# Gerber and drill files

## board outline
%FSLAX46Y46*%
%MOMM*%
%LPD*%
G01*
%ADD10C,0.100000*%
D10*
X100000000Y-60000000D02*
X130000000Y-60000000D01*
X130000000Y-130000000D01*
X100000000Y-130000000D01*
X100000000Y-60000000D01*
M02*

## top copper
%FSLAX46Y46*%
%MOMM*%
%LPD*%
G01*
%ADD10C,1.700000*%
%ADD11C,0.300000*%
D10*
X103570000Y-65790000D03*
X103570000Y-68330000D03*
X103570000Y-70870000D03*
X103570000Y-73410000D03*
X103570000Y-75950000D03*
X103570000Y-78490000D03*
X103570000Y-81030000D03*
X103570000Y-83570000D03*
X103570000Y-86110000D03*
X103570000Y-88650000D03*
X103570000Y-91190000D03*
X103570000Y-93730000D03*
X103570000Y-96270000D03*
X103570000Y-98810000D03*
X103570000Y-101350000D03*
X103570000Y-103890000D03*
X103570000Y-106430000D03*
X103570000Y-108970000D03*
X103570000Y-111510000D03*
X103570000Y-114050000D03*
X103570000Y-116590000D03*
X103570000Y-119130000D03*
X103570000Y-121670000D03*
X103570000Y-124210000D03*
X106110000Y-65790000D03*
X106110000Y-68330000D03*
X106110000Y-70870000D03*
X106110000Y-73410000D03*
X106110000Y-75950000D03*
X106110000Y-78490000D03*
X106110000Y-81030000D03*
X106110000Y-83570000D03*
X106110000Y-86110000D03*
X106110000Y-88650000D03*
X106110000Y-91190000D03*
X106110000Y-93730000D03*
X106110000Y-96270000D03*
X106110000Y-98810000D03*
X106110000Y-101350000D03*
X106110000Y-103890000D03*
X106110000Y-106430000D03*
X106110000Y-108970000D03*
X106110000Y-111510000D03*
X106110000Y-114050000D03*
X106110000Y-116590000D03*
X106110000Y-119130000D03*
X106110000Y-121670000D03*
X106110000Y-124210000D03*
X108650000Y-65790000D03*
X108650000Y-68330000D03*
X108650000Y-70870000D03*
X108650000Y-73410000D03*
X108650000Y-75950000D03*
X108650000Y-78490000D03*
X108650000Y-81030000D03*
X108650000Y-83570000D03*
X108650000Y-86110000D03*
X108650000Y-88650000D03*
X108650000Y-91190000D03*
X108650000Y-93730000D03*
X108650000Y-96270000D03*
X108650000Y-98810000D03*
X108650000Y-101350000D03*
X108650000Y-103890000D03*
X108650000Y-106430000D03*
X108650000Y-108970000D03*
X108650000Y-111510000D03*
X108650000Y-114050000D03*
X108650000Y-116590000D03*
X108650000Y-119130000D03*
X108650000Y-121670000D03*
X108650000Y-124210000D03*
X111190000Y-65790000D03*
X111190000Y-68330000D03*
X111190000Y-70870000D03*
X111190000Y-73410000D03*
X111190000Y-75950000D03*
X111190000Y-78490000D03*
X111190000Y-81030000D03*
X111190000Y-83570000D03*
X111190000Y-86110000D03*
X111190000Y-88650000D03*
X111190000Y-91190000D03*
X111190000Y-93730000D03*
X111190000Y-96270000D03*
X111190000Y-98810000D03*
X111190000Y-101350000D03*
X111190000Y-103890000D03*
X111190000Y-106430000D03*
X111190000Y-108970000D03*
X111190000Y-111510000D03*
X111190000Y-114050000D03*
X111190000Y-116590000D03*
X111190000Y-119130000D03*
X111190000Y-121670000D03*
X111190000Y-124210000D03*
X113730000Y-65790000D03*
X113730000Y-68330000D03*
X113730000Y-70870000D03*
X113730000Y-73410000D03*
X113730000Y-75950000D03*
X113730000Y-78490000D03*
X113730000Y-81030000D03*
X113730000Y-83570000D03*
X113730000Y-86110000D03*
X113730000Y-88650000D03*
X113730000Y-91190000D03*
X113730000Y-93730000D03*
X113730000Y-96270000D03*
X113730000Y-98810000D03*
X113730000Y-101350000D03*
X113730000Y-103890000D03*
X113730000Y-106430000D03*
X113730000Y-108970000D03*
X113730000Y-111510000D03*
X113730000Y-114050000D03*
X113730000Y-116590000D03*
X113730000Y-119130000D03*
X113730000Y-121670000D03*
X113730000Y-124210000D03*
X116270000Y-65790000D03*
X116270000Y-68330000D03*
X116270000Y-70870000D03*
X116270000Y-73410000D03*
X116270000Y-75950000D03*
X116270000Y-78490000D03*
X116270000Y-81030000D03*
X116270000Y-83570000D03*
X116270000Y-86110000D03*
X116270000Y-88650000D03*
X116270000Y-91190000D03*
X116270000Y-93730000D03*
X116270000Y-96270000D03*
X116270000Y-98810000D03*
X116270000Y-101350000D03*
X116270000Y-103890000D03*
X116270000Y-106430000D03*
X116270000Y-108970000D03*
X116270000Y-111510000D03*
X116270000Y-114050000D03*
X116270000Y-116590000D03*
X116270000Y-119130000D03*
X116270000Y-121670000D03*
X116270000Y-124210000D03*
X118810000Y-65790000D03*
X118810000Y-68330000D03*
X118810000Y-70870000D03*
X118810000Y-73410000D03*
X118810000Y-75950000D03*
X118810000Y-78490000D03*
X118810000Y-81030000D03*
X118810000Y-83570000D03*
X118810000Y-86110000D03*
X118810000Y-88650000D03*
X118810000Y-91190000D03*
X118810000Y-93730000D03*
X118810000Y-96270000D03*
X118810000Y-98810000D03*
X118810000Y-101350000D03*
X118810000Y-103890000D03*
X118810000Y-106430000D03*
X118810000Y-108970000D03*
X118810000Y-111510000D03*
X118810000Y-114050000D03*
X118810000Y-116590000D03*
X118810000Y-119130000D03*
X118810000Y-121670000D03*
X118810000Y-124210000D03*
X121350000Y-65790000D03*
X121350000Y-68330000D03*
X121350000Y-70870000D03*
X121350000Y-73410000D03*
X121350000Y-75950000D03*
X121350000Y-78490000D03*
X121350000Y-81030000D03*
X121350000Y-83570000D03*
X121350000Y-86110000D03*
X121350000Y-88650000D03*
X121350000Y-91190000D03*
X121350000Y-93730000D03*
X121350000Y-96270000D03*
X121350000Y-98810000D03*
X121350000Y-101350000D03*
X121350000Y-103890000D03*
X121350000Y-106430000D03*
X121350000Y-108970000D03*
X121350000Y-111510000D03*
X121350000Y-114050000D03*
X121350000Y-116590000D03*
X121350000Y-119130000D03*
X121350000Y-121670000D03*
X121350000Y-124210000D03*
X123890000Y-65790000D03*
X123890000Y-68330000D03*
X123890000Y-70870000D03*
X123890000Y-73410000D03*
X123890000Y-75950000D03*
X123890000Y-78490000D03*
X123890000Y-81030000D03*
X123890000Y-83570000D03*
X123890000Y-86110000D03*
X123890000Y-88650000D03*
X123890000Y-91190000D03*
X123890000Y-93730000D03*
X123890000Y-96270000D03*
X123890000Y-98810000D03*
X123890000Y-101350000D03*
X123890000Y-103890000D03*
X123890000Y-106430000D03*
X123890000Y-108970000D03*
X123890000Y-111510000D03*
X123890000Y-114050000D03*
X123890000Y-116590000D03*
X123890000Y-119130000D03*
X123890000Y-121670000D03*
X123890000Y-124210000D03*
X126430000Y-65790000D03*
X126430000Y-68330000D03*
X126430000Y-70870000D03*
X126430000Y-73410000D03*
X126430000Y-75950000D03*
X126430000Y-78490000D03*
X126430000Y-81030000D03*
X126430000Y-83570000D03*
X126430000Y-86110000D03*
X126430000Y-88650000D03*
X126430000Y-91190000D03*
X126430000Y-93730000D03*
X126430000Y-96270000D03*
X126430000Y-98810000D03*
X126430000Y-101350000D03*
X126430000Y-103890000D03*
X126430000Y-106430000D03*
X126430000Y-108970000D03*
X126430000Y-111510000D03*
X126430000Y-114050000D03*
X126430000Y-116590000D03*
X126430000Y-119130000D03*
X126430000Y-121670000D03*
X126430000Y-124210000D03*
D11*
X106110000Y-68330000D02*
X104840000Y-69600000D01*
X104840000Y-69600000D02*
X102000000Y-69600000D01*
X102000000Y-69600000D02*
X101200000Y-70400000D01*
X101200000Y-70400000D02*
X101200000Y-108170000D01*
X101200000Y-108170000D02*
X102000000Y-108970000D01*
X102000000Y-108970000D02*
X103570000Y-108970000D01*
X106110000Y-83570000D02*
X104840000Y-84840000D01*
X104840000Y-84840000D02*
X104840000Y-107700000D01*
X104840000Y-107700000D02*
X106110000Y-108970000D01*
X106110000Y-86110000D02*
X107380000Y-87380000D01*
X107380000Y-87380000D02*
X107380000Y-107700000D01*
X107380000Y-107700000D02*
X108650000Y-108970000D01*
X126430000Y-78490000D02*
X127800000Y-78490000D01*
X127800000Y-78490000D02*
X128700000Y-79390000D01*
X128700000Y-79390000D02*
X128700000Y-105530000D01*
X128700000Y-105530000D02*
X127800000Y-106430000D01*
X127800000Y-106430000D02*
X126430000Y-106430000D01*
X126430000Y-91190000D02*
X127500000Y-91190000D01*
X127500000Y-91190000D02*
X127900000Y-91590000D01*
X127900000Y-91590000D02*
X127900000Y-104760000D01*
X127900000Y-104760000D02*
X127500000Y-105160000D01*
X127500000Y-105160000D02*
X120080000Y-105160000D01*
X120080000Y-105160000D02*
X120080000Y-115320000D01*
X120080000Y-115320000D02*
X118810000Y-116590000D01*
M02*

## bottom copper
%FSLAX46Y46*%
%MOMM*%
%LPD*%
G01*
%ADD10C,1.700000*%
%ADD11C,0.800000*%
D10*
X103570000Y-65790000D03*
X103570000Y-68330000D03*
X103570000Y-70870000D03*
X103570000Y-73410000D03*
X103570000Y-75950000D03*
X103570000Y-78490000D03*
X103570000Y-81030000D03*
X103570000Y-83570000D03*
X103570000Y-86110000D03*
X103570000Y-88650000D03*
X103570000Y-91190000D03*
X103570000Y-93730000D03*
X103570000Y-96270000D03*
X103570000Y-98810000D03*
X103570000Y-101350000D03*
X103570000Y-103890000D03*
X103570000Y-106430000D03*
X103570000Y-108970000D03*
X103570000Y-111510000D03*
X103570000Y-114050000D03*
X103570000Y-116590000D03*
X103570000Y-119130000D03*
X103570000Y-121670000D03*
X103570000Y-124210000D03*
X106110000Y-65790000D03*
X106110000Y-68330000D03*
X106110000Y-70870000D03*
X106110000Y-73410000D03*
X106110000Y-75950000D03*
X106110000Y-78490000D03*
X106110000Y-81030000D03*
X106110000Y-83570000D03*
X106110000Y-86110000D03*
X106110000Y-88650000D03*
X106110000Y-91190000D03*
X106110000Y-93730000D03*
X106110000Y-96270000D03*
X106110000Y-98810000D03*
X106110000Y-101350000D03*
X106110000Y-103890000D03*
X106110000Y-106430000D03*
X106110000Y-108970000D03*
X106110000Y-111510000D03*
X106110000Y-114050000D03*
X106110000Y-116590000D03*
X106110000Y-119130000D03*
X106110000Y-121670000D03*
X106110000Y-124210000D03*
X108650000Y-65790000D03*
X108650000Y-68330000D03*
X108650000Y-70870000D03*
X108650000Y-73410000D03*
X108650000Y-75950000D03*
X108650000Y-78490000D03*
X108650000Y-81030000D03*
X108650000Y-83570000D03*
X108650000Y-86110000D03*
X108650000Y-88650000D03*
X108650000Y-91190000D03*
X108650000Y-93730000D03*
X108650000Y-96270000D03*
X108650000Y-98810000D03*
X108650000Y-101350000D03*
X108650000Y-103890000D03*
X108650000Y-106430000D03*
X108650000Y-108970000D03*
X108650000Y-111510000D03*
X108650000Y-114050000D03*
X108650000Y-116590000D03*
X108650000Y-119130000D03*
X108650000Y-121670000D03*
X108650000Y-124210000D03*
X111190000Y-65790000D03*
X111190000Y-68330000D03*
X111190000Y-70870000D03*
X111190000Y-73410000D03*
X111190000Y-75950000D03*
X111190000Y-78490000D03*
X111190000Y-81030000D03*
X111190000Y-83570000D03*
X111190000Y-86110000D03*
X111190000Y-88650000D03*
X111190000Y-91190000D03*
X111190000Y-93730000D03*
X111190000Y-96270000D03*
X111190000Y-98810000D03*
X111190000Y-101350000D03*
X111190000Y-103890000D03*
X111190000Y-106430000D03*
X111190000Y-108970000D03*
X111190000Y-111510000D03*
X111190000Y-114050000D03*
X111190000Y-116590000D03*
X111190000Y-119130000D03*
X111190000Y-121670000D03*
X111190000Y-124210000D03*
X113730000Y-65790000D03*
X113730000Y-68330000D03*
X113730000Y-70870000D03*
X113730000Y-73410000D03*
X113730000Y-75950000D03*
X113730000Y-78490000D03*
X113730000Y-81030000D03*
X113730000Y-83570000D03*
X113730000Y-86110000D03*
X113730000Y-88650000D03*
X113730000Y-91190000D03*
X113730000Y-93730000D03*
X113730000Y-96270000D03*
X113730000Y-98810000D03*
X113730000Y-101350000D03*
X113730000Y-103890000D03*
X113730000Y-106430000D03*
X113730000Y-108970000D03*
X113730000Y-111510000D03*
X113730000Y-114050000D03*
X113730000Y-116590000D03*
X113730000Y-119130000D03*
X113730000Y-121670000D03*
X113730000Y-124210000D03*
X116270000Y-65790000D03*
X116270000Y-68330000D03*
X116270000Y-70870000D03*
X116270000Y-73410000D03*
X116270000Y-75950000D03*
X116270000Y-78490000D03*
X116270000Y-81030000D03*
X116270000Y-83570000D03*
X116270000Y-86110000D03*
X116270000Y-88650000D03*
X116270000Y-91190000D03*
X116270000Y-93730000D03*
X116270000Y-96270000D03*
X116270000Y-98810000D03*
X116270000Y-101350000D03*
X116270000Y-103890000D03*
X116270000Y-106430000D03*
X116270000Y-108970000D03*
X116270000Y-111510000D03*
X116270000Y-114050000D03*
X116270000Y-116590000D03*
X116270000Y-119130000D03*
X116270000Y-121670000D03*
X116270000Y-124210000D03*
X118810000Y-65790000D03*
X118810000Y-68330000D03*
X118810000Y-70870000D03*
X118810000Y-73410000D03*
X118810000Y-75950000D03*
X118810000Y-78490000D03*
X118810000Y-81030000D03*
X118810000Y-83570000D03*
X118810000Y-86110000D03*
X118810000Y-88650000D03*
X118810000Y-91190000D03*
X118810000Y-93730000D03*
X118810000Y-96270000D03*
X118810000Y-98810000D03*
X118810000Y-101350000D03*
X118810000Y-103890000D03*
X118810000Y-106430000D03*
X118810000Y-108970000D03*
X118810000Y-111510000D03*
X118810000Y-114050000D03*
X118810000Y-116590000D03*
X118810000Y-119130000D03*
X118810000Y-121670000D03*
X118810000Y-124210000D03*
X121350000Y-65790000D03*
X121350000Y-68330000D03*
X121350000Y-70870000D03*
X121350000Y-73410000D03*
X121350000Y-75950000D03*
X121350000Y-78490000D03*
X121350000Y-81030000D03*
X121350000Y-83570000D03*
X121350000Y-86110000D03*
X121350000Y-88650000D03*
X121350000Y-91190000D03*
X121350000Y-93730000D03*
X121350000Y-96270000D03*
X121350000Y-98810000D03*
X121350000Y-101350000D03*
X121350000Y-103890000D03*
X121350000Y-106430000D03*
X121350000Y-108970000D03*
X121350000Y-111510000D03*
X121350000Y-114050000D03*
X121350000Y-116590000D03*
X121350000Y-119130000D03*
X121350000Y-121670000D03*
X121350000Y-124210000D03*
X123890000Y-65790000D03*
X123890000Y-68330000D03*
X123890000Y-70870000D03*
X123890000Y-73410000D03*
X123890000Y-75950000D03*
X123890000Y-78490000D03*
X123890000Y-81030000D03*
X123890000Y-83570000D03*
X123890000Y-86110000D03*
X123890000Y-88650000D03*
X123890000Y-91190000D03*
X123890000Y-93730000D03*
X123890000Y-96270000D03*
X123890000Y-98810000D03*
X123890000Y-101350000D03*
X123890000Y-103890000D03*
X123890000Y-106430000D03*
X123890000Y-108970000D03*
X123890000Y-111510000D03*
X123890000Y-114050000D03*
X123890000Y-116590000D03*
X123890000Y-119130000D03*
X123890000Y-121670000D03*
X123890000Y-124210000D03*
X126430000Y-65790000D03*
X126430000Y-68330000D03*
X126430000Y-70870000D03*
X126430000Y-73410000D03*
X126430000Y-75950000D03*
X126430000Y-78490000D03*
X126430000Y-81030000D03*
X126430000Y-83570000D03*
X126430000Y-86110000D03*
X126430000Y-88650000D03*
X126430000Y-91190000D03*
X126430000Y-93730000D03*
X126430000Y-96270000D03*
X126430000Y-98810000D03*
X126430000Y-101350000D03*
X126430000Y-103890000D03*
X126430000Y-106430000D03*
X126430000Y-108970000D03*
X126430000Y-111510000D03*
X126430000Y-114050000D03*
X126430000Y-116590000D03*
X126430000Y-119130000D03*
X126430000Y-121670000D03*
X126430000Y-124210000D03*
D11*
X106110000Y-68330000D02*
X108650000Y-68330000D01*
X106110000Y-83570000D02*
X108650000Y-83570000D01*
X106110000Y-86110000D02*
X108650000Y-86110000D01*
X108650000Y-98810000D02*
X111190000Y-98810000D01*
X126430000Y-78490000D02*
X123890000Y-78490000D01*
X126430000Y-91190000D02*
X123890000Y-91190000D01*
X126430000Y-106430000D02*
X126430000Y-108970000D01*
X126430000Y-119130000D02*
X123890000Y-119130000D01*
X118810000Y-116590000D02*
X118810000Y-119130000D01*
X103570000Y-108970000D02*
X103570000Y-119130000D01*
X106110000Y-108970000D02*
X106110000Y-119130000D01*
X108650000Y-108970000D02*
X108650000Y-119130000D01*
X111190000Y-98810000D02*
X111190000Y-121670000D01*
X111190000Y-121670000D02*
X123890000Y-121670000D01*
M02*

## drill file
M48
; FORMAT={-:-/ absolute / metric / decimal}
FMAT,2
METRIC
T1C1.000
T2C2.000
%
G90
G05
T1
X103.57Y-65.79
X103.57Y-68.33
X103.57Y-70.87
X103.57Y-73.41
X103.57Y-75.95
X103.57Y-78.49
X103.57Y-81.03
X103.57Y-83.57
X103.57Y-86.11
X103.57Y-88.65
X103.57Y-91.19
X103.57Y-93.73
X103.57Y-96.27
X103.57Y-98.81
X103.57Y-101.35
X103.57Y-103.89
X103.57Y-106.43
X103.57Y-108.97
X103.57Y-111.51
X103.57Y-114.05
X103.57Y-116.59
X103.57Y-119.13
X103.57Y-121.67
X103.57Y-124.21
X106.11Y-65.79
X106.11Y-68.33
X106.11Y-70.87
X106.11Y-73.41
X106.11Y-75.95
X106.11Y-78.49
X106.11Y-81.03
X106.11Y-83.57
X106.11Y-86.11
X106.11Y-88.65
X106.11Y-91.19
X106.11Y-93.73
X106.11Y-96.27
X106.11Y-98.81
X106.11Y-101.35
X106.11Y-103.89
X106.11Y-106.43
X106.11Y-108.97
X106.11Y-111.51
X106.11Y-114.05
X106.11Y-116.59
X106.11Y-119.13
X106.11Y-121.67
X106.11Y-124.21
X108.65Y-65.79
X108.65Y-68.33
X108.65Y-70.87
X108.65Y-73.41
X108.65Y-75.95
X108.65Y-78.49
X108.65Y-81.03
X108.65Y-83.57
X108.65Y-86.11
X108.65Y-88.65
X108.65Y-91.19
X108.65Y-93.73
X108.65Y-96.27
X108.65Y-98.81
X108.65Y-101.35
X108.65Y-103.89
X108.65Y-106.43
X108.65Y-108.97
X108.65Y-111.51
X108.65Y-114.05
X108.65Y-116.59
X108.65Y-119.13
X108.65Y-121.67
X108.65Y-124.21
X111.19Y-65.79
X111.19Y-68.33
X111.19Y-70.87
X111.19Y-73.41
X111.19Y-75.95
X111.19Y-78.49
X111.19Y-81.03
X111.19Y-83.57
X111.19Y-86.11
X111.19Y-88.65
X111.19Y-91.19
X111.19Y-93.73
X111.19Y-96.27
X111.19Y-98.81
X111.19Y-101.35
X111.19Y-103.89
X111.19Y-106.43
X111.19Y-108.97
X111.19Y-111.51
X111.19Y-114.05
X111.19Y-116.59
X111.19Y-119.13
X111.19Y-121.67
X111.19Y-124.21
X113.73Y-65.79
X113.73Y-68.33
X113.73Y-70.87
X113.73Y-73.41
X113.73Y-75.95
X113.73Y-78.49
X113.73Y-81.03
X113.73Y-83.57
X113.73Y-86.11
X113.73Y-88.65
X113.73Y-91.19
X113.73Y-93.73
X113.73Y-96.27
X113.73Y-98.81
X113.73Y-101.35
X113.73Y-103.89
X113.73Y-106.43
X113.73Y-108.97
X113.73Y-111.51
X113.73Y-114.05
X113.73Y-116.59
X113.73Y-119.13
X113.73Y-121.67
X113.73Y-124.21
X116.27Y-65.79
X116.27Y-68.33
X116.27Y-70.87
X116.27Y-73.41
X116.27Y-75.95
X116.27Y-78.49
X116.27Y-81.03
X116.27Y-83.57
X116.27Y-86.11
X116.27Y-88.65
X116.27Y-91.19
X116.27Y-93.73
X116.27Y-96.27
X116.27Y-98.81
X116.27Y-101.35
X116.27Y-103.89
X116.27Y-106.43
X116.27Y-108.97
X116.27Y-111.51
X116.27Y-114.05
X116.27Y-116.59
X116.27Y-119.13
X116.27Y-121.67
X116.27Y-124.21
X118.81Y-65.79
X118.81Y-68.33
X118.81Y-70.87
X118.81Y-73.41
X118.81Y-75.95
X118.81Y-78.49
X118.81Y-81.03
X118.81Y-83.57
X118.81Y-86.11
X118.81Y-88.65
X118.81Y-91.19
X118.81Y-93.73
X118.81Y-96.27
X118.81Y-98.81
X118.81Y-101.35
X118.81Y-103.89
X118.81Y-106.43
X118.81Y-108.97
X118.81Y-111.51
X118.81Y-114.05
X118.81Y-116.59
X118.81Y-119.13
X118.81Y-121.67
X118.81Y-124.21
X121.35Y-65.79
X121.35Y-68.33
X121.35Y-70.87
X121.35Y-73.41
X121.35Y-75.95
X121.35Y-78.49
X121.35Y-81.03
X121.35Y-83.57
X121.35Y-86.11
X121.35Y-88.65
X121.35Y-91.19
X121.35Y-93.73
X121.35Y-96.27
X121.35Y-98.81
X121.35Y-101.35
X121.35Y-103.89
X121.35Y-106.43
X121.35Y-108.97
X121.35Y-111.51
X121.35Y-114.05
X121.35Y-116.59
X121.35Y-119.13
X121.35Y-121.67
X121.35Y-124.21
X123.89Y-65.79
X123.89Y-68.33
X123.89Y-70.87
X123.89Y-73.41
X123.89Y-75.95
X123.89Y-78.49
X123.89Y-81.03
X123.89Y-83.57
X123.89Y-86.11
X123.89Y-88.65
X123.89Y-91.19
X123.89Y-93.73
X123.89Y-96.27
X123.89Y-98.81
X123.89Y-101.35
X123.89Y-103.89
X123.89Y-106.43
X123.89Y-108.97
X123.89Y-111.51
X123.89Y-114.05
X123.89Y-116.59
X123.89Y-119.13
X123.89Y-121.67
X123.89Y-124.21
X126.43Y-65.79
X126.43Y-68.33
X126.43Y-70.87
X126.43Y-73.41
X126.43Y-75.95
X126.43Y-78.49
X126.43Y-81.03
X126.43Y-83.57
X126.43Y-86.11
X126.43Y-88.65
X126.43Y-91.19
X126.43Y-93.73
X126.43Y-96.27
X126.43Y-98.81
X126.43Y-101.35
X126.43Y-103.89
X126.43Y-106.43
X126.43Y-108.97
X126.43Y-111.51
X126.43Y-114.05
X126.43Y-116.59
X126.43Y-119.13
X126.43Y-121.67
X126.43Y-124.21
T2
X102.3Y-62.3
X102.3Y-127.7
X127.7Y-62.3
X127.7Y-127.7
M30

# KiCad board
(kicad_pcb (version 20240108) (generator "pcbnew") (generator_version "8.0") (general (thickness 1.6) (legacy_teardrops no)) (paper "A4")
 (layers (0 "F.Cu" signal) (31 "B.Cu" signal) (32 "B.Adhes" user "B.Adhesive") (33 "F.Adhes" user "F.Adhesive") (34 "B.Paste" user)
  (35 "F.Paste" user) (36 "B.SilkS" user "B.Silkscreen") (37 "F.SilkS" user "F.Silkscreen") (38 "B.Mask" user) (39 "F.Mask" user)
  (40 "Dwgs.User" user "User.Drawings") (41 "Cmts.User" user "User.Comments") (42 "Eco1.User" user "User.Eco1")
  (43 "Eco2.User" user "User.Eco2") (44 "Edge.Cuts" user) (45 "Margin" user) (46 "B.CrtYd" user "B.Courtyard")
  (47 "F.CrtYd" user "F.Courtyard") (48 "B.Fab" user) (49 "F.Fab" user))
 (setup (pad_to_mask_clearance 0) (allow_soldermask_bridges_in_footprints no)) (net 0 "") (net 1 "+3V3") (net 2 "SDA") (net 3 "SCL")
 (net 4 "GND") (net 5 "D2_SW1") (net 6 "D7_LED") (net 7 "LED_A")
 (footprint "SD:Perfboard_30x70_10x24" (layer "F.Cu") (at 100 60)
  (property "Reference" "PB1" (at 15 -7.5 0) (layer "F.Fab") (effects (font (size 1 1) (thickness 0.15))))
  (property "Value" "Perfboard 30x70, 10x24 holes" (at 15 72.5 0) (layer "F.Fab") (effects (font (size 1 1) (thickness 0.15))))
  (pad "A1" thru_hole circle (at 3.57 5.79) (size 1.7 1.7) (drill 1) (layers "*.Cu" "*.Mask") (remove_unused_layers no))
  (pad "A2" thru_hole circle (at 3.57 8.33) (size 1.7 1.7) (drill 1) (layers "*.Cu" "*.Mask") (remove_unused_layers no))
  (pad "A3" thru_hole circle (at 3.57 10.87) (size 1.7 1.7) (drill 1) (layers "*.Cu" "*.Mask") (remove_unused_layers no))
  (pad "A4" thru_hole circle (at 3.57 13.41) (size 1.7 1.7) (drill 1) (layers "*.Cu" "*.Mask") (remove_unused_layers no))
  (pad "A5" thru_hole circle (at 3.57 15.95) (size 1.7 1.7) (drill 1) (layers "*.Cu" "*.Mask") (remove_unused_layers no))
  (pad "A6" thru_hole circle (at 3.57 18.49) (size 1.7 1.7) (drill 1) (layers "*.Cu" "*.Mask") (remove_unused_layers no))
  (pad "A7" thru_hole circle (at 3.57 21.03) (size 1.7 1.7) (drill 1) (layers "*.Cu" "*.Mask") (remove_unused_layers no))
  (pad "A8" thru_hole circle (at 3.57 23.57) (size 1.7 1.7) (drill 1) (layers "*.Cu" "*.Mask") (remove_unused_layers no))
  (pad "A9" thru_hole circle (at 3.57 26.11) (size 1.7 1.7) (drill 1) (layers "*.Cu" "*.Mask") (remove_unused_layers no))
  (pad "A10" thru_hole circle (at 3.57 28.65) (size 1.7 1.7) (drill 1) (layers "*.Cu" "*.Mask") (remove_unused_layers no))
  (pad "A11" thru_hole circle (at 3.57 31.19) (size 1.7 1.7) (drill 1) (layers "*.Cu" "*.Mask") (remove_unused_layers no))
  (pad "A12" thru_hole circle (at 3.57 33.73) (size 1.7 1.7) (drill 1) (layers "*.Cu" "*.Mask") (remove_unused_layers no))
  (pad "A13" thru_hole circle (at 3.57 36.27) (size 1.7 1.7) (drill 1) (layers "*.Cu" "*.Mask") (remove_unused_layers no))
  (pad "A14" thru_hole circle (at 3.57 38.81) (size 1.7 1.7) (drill 1) (layers "*.Cu" "*.Mask") (remove_unused_layers no))
  (pad "A15" thru_hole circle (at 3.57 41.35) (size 1.7 1.7) (drill 1) (layers "*.Cu" "*.Mask") (remove_unused_layers no))
  (pad "A16" thru_hole circle (at 3.57 43.89) (size 1.7 1.7) (drill 1) (layers "*.Cu" "*.Mask") (remove_unused_layers no))
  (pad "A17" thru_hole circle (at 3.57 46.43) (size 1.7 1.7) (drill 1) (layers "*.Cu" "*.Mask") (remove_unused_layers no))
  (pad "A18" thru_hole circle (at 3.57 48.97) (size 1.7 1.7) (drill 1) (layers "*.Cu" "*.Mask") (remove_unused_layers no) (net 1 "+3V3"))
  (pad "A19" thru_hole circle (at 3.57 51.51) (size 1.7 1.7) (drill 1) (layers "*.Cu" "*.Mask") (remove_unused_layers no) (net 1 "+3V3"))
  (pad "A20" thru_hole circle (at 3.57 54.05) (size 1.7 1.7) (drill 1) (layers "*.Cu" "*.Mask") (remove_unused_layers no) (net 1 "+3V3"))
  (pad "A21" thru_hole circle (at 3.57 56.59) (size 1.7 1.7) (drill 1) (layers "*.Cu" "*.Mask") (remove_unused_layers no) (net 1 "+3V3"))
  (pad "A22" thru_hole circle (at 3.57 59.13) (size 1.7 1.7) (drill 1) (layers "*.Cu" "*.Mask") (remove_unused_layers no) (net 1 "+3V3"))
  (pad "A23" thru_hole circle (at 3.57 61.67) (size 1.7 1.7) (drill 1) (layers "*.Cu" "*.Mask") (remove_unused_layers no))
  (pad "A24" thru_hole circle (at 3.57 64.21) (size 1.7 1.7) (drill 1) (layers "*.Cu" "*.Mask") (remove_unused_layers no))
  (pad "B1" thru_hole circle (at 6.11 5.79) (size 1.7 1.7) (drill 1) (layers "*.Cu" "*.Mask") (remove_unused_layers no))
  (pad "B2" thru_hole circle (at 6.11 8.33) (size 1.7 1.7) (drill 1) (layers "*.Cu" "*.Mask") (remove_unused_layers no) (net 1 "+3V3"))
  (pad "B3" thru_hole circle (at 6.11 10.87) (size 1.7 1.7) (drill 1) (layers "*.Cu" "*.Mask") (remove_unused_layers no))
  (pad "B4" thru_hole circle (at 6.11 13.41) (size 1.7 1.7) (drill 1) (layers "*.Cu" "*.Mask") (remove_unused_layers no))
  (pad "B5" thru_hole circle (at 6.11 15.95) (size 1.7 1.7) (drill 1) (layers "*.Cu" "*.Mask") (remove_unused_layers no))
  (pad "B6" thru_hole circle (at 6.11 18.49) (size 1.7 1.7) (drill 1) (layers "*.Cu" "*.Mask") (remove_unused_layers no))
  (pad "B7" thru_hole circle (at 6.11 21.03) (size 1.7 1.7) (drill 1) (layers "*.Cu" "*.Mask") (remove_unused_layers no))
  (pad "B8" thru_hole circle (at 6.11 23.57) (size 1.7 1.7) (drill 1) (layers "*.Cu" "*.Mask") (remove_unused_layers no) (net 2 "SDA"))
  (pad "B9" thru_hole circle (at 6.11 26.11) (size 1.7 1.7) (drill 1) (layers "*.Cu" "*.Mask") (remove_unused_layers no) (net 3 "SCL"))
  (pad "B10" thru_hole circle (at 6.11 28.65) (size 1.7 1.7) (drill 1) (layers "*.Cu" "*.Mask") (remove_unused_layers no))
  (pad "B11" thru_hole circle (at 6.11 31.19) (size 1.7 1.7) (drill 1) (layers "*.Cu" "*.Mask") (remove_unused_layers no))
  (pad "B12" thru_hole circle (at 6.11 33.73) (size 1.7 1.7) (drill 1) (layers "*.Cu" "*.Mask") (remove_unused_layers no))
  (pad "B13" thru_hole circle (at 6.11 36.27) (size 1.7 1.7) (drill 1) (layers "*.Cu" "*.Mask") (remove_unused_layers no))
  (pad "B14" thru_hole circle (at 6.11 38.81) (size 1.7 1.7) (drill 1) (layers "*.Cu" "*.Mask") (remove_unused_layers no))
  (pad "B15" thru_hole circle (at 6.11 41.35) (size 1.7 1.7) (drill 1) (layers "*.Cu" "*.Mask") (remove_unused_layers no))
  (pad "B16" thru_hole circle (at 6.11 43.89) (size 1.7 1.7) (drill 1) (layers "*.Cu" "*.Mask") (remove_unused_layers no))
  (pad "B17" thru_hole circle (at 6.11 46.43) (size 1.7 1.7) (drill 1) (layers "*.Cu" "*.Mask") (remove_unused_layers no))
  (pad "B18" thru_hole circle (at 6.11 48.97) (size 1.7 1.7) (drill 1) (layers "*.Cu" "*.Mask") (remove_unused_layers no) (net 2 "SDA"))
  (pad "B19" thru_hole circle (at 6.11 51.51) (size 1.7 1.7) (drill 1) (layers "*.Cu" "*.Mask") (remove_unused_layers no) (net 2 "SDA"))
  (pad "B20" thru_hole circle (at 6.11 54.05) (size 1.7 1.7) (drill 1) (layers "*.Cu" "*.Mask") (remove_unused_layers no) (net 2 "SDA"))
  (pad "B21" thru_hole circle (at 6.11 56.59) (size 1.7 1.7) (drill 1) (layers "*.Cu" "*.Mask") (remove_unused_layers no) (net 2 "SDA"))
  (pad "B22" thru_hole circle (at 6.11 59.13) (size 1.7 1.7) (drill 1) (layers "*.Cu" "*.Mask") (remove_unused_layers no) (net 2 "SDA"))
  (pad "B23" thru_hole circle (at 6.11 61.67) (size 1.7 1.7) (drill 1) (layers "*.Cu" "*.Mask") (remove_unused_layers no))
  (pad "B24" thru_hole circle (at 6.11 64.21) (size 1.7 1.7) (drill 1) (layers "*.Cu" "*.Mask") (remove_unused_layers no))
  (pad "C1" thru_hole circle (at 8.65 5.79) (size 1.7 1.7) (drill 1) (layers "*.Cu" "*.Mask") (remove_unused_layers no))
  (pad "C2" thru_hole circle (at 8.65 8.33) (size 1.7 1.7) (drill 1) (layers "*.Cu" "*.Mask") (remove_unused_layers no) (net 1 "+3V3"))
  (pad "C3" thru_hole circle (at 8.65 10.87) (size 1.7 1.7) (drill 1) (layers "*.Cu" "*.Mask") (remove_unused_layers no))
  (pad "C4" thru_hole circle (at 8.65 13.41) (size 1.7 1.7) (drill 1) (layers "*.Cu" "*.Mask") (remove_unused_layers no))
  (pad "C5" thru_hole circle (at 8.65 15.95) (size 1.7 1.7) (drill 1) (layers "*.Cu" "*.Mask") (remove_unused_layers no))
  (pad "C6" thru_hole circle (at 8.65 18.49) (size 1.7 1.7) (drill 1) (layers "*.Cu" "*.Mask") (remove_unused_layers no))
  (pad "C7" thru_hole circle (at 8.65 21.03) (size 1.7 1.7) (drill 1) (layers "*.Cu" "*.Mask") (remove_unused_layers no))
  (pad "C8" thru_hole circle (at 8.65 23.57) (size 1.7 1.7) (drill 1) (layers "*.Cu" "*.Mask") (remove_unused_layers no) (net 2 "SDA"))
  (pad "C9" thru_hole circle (at 8.65 26.11) (size 1.7 1.7) (drill 1) (layers "*.Cu" "*.Mask") (remove_unused_layers no) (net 3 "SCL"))
  (pad "C10" thru_hole circle (at 8.65 28.65) (size 1.7 1.7) (drill 1) (layers "*.Cu" "*.Mask") (remove_unused_layers no))
  (pad "C11" thru_hole circle (at 8.65 31.19) (size 1.7 1.7) (drill 1) (layers "*.Cu" "*.Mask") (remove_unused_layers no))
  (pad "C12" thru_hole circle (at 8.65 33.73) (size 1.7 1.7) (drill 1) (layers "*.Cu" "*.Mask") (remove_unused_layers no))
  (pad "C13" thru_hole circle (at 8.65 36.27) (size 1.7 1.7) (drill 1) (layers "*.Cu" "*.Mask") (remove_unused_layers no))
  (pad "C14" thru_hole circle (at 8.65 38.81) (size 1.7 1.7) (drill 1) (layers "*.Cu" "*.Mask") (remove_unused_layers no) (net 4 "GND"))
  (pad "C15" thru_hole circle (at 8.65 41.35) (size 1.7 1.7) (drill 1) (layers "*.Cu" "*.Mask") (remove_unused_layers no))
  (pad "C16" thru_hole circle (at 8.65 43.89) (size 1.7 1.7) (drill 1) (layers "*.Cu" "*.Mask") (remove_unused_layers no))
  (pad "C17" thru_hole circle (at 8.65 46.43) (size 1.7 1.7) (drill 1) (layers "*.Cu" "*.Mask") (remove_unused_layers no))
  (pad "C18" thru_hole circle (at 8.65 48.97) (size 1.7 1.7) (drill 1) (layers "*.Cu" "*.Mask") (remove_unused_layers no) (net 3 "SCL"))
  (pad "C19" thru_hole circle (at 8.65 51.51) (size 1.7 1.7) (drill 1) (layers "*.Cu" "*.Mask") (remove_unused_layers no) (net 3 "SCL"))
  (pad "C20" thru_hole circle (at 8.65 54.05) (size 1.7 1.7) (drill 1) (layers "*.Cu" "*.Mask") (remove_unused_layers no) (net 3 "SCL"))
  (pad "C21" thru_hole circle (at 8.65 56.59) (size 1.7 1.7) (drill 1) (layers "*.Cu" "*.Mask") (remove_unused_layers no) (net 3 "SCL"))
  (pad "C22" thru_hole circle (at 8.65 59.13) (size 1.7 1.7) (drill 1) (layers "*.Cu" "*.Mask") (remove_unused_layers no) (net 3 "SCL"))
  (pad "C23" thru_hole circle (at 8.65 61.67) (size 1.7 1.7) (drill 1) (layers "*.Cu" "*.Mask") (remove_unused_layers no))
  (pad "C24" thru_hole circle (at 8.65 64.21) (size 1.7 1.7) (drill 1) (layers "*.Cu" "*.Mask") (remove_unused_layers no))
  (pad "D1" thru_hole circle (at 11.19 5.79) (size 1.7 1.7) (drill 1) (layers "*.Cu" "*.Mask") (remove_unused_layers no))
  (pad "D2" thru_hole circle (at 11.19 8.33) (size 1.7 1.7) (drill 1) (layers "*.Cu" "*.Mask") (remove_unused_layers no))
  (pad "D3" thru_hole circle (at 11.19 10.87) (size 1.7 1.7) (drill 1) (layers "*.Cu" "*.Mask") (remove_unused_layers no))
  (pad "D4" thru_hole circle (at 11.19 13.41) (size 1.7 1.7) (drill 1) (layers "*.Cu" "*.Mask") (remove_unused_layers no))
  (pad "D5" thru_hole circle (at 11.19 15.95) (size 1.7 1.7) (drill 1) (layers "*.Cu" "*.Mask") (remove_unused_layers no))
  (pad "D6" thru_hole circle (at 11.19 18.49) (size 1.7 1.7) (drill 1) (layers "*.Cu" "*.Mask") (remove_unused_layers no))
  (pad "D7" thru_hole circle (at 11.19 21.03) (size 1.7 1.7) (drill 1) (layers "*.Cu" "*.Mask") (remove_unused_layers no))
  (pad "D8" thru_hole circle (at 11.19 23.57) (size 1.7 1.7) (drill 1) (layers "*.Cu" "*.Mask") (remove_unused_layers no))
  (pad "D9" thru_hole circle (at 11.19 26.11) (size 1.7 1.7) (drill 1) (layers "*.Cu" "*.Mask") (remove_unused_layers no))
  (pad "D10" thru_hole circle (at 11.19 28.65) (size 1.7 1.7) (drill 1) (layers "*.Cu" "*.Mask") (remove_unused_layers no))
  (pad "D11" thru_hole circle (at 11.19 31.19) (size 1.7 1.7) (drill 1) (layers "*.Cu" "*.Mask") (remove_unused_layers no))
  (pad "D12" thru_hole circle (at 11.19 33.73) (size 1.7 1.7) (drill 1) (layers "*.Cu" "*.Mask") (remove_unused_layers no))
  (pad "D13" thru_hole circle (at 11.19 36.27) (size 1.7 1.7) (drill 1) (layers "*.Cu" "*.Mask") (remove_unused_layers no))
  (pad "D14" thru_hole circle (at 11.19 38.81) (size 1.7 1.7) (drill 1) (layers "*.Cu" "*.Mask") (remove_unused_layers no) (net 4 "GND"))
  (pad "D15" thru_hole circle (at 11.19 41.35) (size 1.7 1.7) (drill 1) (layers "*.Cu" "*.Mask") (remove_unused_layers no) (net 4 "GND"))
  (pad "D16" thru_hole circle (at 11.19 43.89) (size 1.7 1.7) (drill 1) (layers "*.Cu" "*.Mask") (remove_unused_layers no) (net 4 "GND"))
  (pad "D17" thru_hole circle (at 11.19 46.43) (size 1.7 1.7) (drill 1) (layers "*.Cu" "*.Mask") (remove_unused_layers no) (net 4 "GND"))
  (pad "D18" thru_hole circle (at 11.19 48.97) (size 1.7 1.7) (drill 1) (layers "*.Cu" "*.Mask") (remove_unused_layers no) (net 4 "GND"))
  (pad "D19" thru_hole circle (at 11.19 51.51) (size 1.7 1.7) (drill 1) (layers "*.Cu" "*.Mask") (remove_unused_layers no) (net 4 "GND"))
  (pad "D20" thru_hole circle (at 11.19 54.05) (size 1.7 1.7) (drill 1) (layers "*.Cu" "*.Mask") (remove_unused_layers no) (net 4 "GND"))
  (pad "D21" thru_hole circle (at 11.19 56.59) (size 1.7 1.7) (drill 1) (layers "*.Cu" "*.Mask") (remove_unused_layers no) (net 4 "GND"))
  (pad "D22" thru_hole circle (at 11.19 59.13) (size 1.7 1.7) (drill 1) (layers "*.Cu" "*.Mask") (remove_unused_layers no) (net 4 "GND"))
  (pad "D23" thru_hole circle (at 11.19 61.67) (size 1.7 1.7) (drill 1) (layers "*.Cu" "*.Mask") (remove_unused_layers no) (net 4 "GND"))
  (pad "D24" thru_hole circle (at 11.19 64.21) (size 1.7 1.7) (drill 1) (layers "*.Cu" "*.Mask") (remove_unused_layers no))
  (pad "E1" thru_hole circle (at 13.73 5.79) (size 1.7 1.7) (drill 1) (layers "*.Cu" "*.Mask") (remove_unused_layers no))
  (pad "E2" thru_hole circle (at 13.73 8.33) (size 1.7 1.7) (drill 1) (layers "*.Cu" "*.Mask") (remove_unused_layers no))
  (pad "E3" thru_hole circle (at 13.73 10.87) (size 1.7 1.7) (drill 1) (layers "*.Cu" "*.Mask") (remove_unused_layers no))
  (pad "E4" thru_hole circle (at 13.73 13.41) (size 1.7 1.7) (drill 1) (layers "*.Cu" "*.Mask") (remove_unused_layers no))
  (pad "E5" thru_hole circle (at 13.73 15.95) (size 1.7 1.7) (drill 1) (layers "*.Cu" "*.Mask") (remove_unused_layers no))
  (pad "E6" thru_hole circle (at 13.73 18.49) (size 1.7 1.7) (drill 1) (layers "*.Cu" "*.Mask") (remove_unused_layers no))
  (pad "E7" thru_hole circle (at 13.73 21.03) (size 1.7 1.7) (drill 1) (layers "*.Cu" "*.Mask") (remove_unused_layers no))
  (pad "E8" thru_hole circle (at 13.73 23.57) (size 1.7 1.7) (drill 1) (layers "*.Cu" "*.Mask") (remove_unused_layers no))
  (pad "E9" thru_hole circle (at 13.73 26.11) (size 1.7 1.7) (drill 1) (layers "*.Cu" "*.Mask") (remove_unused_layers no))
  (pad "E10" thru_hole circle (at 13.73 28.65) (size 1.7 1.7) (drill 1) (layers "*.Cu" "*.Mask") (remove_unused_layers no))
  (pad "E11" thru_hole circle (at 13.73 31.19) (size 1.7 1.7) (drill 1) (layers "*.Cu" "*.Mask") (remove_unused_layers no))
  (pad "E12" thru_hole circle (at 13.73 33.73) (size 1.7 1.7) (drill 1) (layers "*.Cu" "*.Mask") (remove_unused_layers no))
  (pad "E13" thru_hole circle (at 13.73 36.27) (size 1.7 1.7) (drill 1) (layers "*.Cu" "*.Mask") (remove_unused_layers no))
  (pad "E14" thru_hole circle (at 13.73 38.81) (size 1.7 1.7) (drill 1) (layers "*.Cu" "*.Mask") (remove_unused_layers no))
  (pad "E15" thru_hole circle (at 13.73 41.35) (size 1.7 1.7) (drill 1) (layers "*.Cu" "*.Mask") (remove_unused_layers no))
  (pad "E16" thru_hole circle (at 13.73 43.89) (size 1.7 1.7) (drill 1) (layers "*.Cu" "*.Mask") (remove_unused_layers no))
  (pad "E17" thru_hole circle (at 13.73 46.43) (size 1.7 1.7) (drill 1) (layers "*.Cu" "*.Mask") (remove_unused_layers no))
  (pad "E18" thru_hole circle (at 13.73 48.97) (size 1.7 1.7) (drill 1) (layers "*.Cu" "*.Mask") (remove_unused_layers no))
  (pad "E19" thru_hole circle (at 13.73 51.51) (size 1.7 1.7) (drill 1) (layers "*.Cu" "*.Mask") (remove_unused_layers no))
  (pad "E20" thru_hole circle (at 13.73 54.05) (size 1.7 1.7) (drill 1) (layers "*.Cu" "*.Mask") (remove_unused_layers no))
  (pad "E21" thru_hole circle (at 13.73 56.59) (size 1.7 1.7) (drill 1) (layers "*.Cu" "*.Mask") (remove_unused_layers no))
  (pad "E22" thru_hole circle (at 13.73 59.13) (size 1.7 1.7) (drill 1) (layers "*.Cu" "*.Mask") (remove_unused_layers no))
  (pad "E23" thru_hole circle (at 13.73 61.67) (size 1.7 1.7) (drill 1) (layers "*.Cu" "*.Mask") (remove_unused_layers no) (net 4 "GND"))
  (pad "E24" thru_hole circle (at 13.73 64.21) (size 1.7 1.7) (drill 1) (layers "*.Cu" "*.Mask") (remove_unused_layers no))
  (pad "F1" thru_hole circle (at 16.27 5.79) (size 1.7 1.7) (drill 1) (layers "*.Cu" "*.Mask") (remove_unused_layers no))
  (pad "F2" thru_hole circle (at 16.27 8.33) (size 1.7 1.7) (drill 1) (layers "*.Cu" "*.Mask") (remove_unused_layers no))
  (pad "F3" thru_hole circle (at 16.27 10.87) (size 1.7 1.7) (drill 1) (layers "*.Cu" "*.Mask") (remove_unused_layers no))
  (pad "F4" thru_hole circle (at 16.27 13.41) (size 1.7 1.7) (drill 1) (layers "*.Cu" "*.Mask") (remove_unused_layers no))
  (pad "F5" thru_hole circle (at 16.27 15.95) (size 1.7 1.7) (drill 1) (layers "*.Cu" "*.Mask") (remove_unused_layers no))
  (pad "F6" thru_hole circle (at 16.27 18.49) (size 1.7 1.7) (drill 1) (layers "*.Cu" "*.Mask") (remove_unused_layers no))
  (pad "F7" thru_hole circle (at 16.27 21.03) (size 1.7 1.7) (drill 1) (layers "*.Cu" "*.Mask") (remove_unused_layers no))
  (pad "F8" thru_hole circle (at 16.27 23.57) (size 1.7 1.7) (drill 1) (layers "*.Cu" "*.Mask") (remove_unused_layers no))
  (pad "F9" thru_hole circle (at 16.27 26.11) (size 1.7 1.7) (drill 1) (layers "*.Cu" "*.Mask") (remove_unused_layers no))
  (pad "F10" thru_hole circle (at 16.27 28.65) (size 1.7 1.7) (drill 1) (layers "*.Cu" "*.Mask") (remove_unused_layers no))
  (pad "F11" thru_hole circle (at 16.27 31.19) (size 1.7 1.7) (drill 1) (layers "*.Cu" "*.Mask") (remove_unused_layers no))
  (pad "F12" thru_hole circle (at 16.27 33.73) (size 1.7 1.7) (drill 1) (layers "*.Cu" "*.Mask") (remove_unused_layers no))
  (pad "F13" thru_hole circle (at 16.27 36.27) (size 1.7 1.7) (drill 1) (layers "*.Cu" "*.Mask") (remove_unused_layers no))
  (pad "F14" thru_hole circle (at 16.27 38.81) (size 1.7 1.7) (drill 1) (layers "*.Cu" "*.Mask") (remove_unused_layers no))
  (pad "F15" thru_hole circle (at 16.27 41.35) (size 1.7 1.7) (drill 1) (layers "*.Cu" "*.Mask") (remove_unused_layers no))
  (pad "F16" thru_hole circle (at 16.27 43.89) (size 1.7 1.7) (drill 1) (layers "*.Cu" "*.Mask") (remove_unused_layers no))
  (pad "F17" thru_hole circle (at 16.27 46.43) (size 1.7 1.7) (drill 1) (layers "*.Cu" "*.Mask") (remove_unused_layers no))
  (pad "F18" thru_hole circle (at 16.27 48.97) (size 1.7 1.7) (drill 1) (layers "*.Cu" "*.Mask") (remove_unused_layers no))
  (pad "F19" thru_hole circle (at 16.27 51.51) (size 1.7 1.7) (drill 1) (layers "*.Cu" "*.Mask") (remove_unused_layers no))
  (pad "F20" thru_hole circle (at 16.27 54.05) (size 1.7 1.7) (drill 1) (layers "*.Cu" "*.Mask") (remove_unused_layers no))
  (pad "F21" thru_hole circle (at 16.27 56.59) (size 1.7 1.7) (drill 1) (layers "*.Cu" "*.Mask") (remove_unused_layers no))
  (pad "F22" thru_hole circle (at 16.27 59.13) (size 1.7 1.7) (drill 1) (layers "*.Cu" "*.Mask") (remove_unused_layers no))
  (pad "F23" thru_hole circle (at 16.27 61.67) (size 1.7 1.7) (drill 1) (layers "*.Cu" "*.Mask") (remove_unused_layers no) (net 4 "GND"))
  (pad "F24" thru_hole circle (at 16.27 64.21) (size 1.7 1.7) (drill 1) (layers "*.Cu" "*.Mask") (remove_unused_layers no))
  (pad "G1" thru_hole circle (at 18.81 5.79) (size 1.7 1.7) (drill 1) (layers "*.Cu" "*.Mask") (remove_unused_layers no))
  (pad "G2" thru_hole circle (at 18.81 8.33) (size 1.7 1.7) (drill 1) (layers "*.Cu" "*.Mask") (remove_unused_layers no))
  (pad "G3" thru_hole circle (at 18.81 10.87) (size 1.7 1.7) (drill 1) (layers "*.Cu" "*.Mask") (remove_unused_layers no))
  (pad "G4" thru_hole circle (at 18.81 13.41) (size 1.7 1.7) (drill 1) (layers "*.Cu" "*.Mask") (remove_unused_layers no))
  (pad "G5" thru_hole circle (at 18.81 15.95) (size 1.7 1.7) (drill 1) (layers "*.Cu" "*.Mask") (remove_unused_layers no))
  (pad "G6" thru_hole circle (at 18.81 18.49) (size 1.7 1.7) (drill 1) (layers "*.Cu" "*.Mask") (remove_unused_layers no))
  (pad "G7" thru_hole circle (at 18.81 21.03) (size 1.7 1.7) (drill 1) (layers "*.Cu" "*.Mask") (remove_unused_layers no))
  (pad "G8" thru_hole circle (at 18.81 23.57) (size 1.7 1.7) (drill 1) (layers "*.Cu" "*.Mask") (remove_unused_layers no))
  (pad "G9" thru_hole circle (at 18.81 26.11) (size 1.7 1.7) (drill 1) (layers "*.Cu" "*.Mask") (remove_unused_layers no))
  (pad "G10" thru_hole circle (at 18.81 28.65) (size 1.7 1.7) (drill 1) (layers "*.Cu" "*.Mask") (remove_unused_layers no))
  (pad "G11" thru_hole circle (at 18.81 31.19) (size 1.7 1.7) (drill 1) (layers "*.Cu" "*.Mask") (remove_unused_layers no))
  (pad "G12" thru_hole circle (at 18.81 33.73) (size 1.7 1.7) (drill 1) (layers "*.Cu" "*.Mask") (remove_unused_layers no))
  (pad "G13" thru_hole circle (at 18.81 36.27) (size 1.7 1.7) (drill 1) (layers "*.Cu" "*.Mask") (remove_unused_layers no))
  (pad "G14" thru_hole circle (at 18.81 38.81) (size 1.7 1.7) (drill 1) (layers "*.Cu" "*.Mask") (remove_unused_layers no))
  (pad "G15" thru_hole circle (at 18.81 41.35) (size 1.7 1.7) (drill 1) (layers "*.Cu" "*.Mask") (remove_unused_layers no))
  (pad "G16" thru_hole circle (at 18.81 43.89) (size 1.7 1.7) (drill 1) (layers "*.Cu" "*.Mask") (remove_unused_layers no))
  (pad "G17" thru_hole circle (at 18.81 46.43) (size 1.7 1.7) (drill 1) (layers "*.Cu" "*.Mask") (remove_unused_layers no))
  (pad "G18" thru_hole circle (at 18.81 48.97) (size 1.7 1.7) (drill 1) (layers "*.Cu" "*.Mask") (remove_unused_layers no))
  (pad "G19" thru_hole circle (at 18.81 51.51) (size 1.7 1.7) (drill 1) (layers "*.Cu" "*.Mask") (remove_unused_layers no))
  (pad "G20" thru_hole circle (at 18.81 54.05) (size 1.7 1.7) (drill 1) (layers "*.Cu" "*.Mask") (remove_unused_layers no))
  (pad "G21" thru_hole circle (at 18.81 56.59) (size 1.7 1.7) (drill 1) (layers "*.Cu" "*.Mask") (remove_unused_layers no) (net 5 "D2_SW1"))
  (pad "G22" thru_hole circle (at 18.81 59.13) (size 1.7 1.7) (drill 1) (layers "*.Cu" "*.Mask") (remove_unused_layers no) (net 5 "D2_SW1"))
  (pad "G23" thru_hole circle (at 18.81 61.67) (size 1.7 1.7) (drill 1) (layers "*.Cu" "*.Mask") (remove_unused_layers no) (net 4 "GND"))
  (pad "G24" thru_hole circle (at 18.81 64.21) (size 1.7 1.7) (drill 1) (layers "*.Cu" "*.Mask") (remove_unused_layers no))
  (pad "H1" thru_hole circle (at 21.35 5.79) (size 1.7 1.7) (drill 1) (layers "*.Cu" "*.Mask") (remove_unused_layers no))
  (pad "H2" thru_hole circle (at 21.35 8.33) (size 1.7 1.7) (drill 1) (layers "*.Cu" "*.Mask") (remove_unused_layers no))
  (pad "H3" thru_hole circle (at 21.35 10.87) (size 1.7 1.7) (drill 1) (layers "*.Cu" "*.Mask") (remove_unused_layers no))
  (pad "H4" thru_hole circle (at 21.35 13.41) (size 1.7 1.7) (drill 1) (layers "*.Cu" "*.Mask") (remove_unused_layers no))
  (pad "H5" thru_hole circle (at 21.35 15.95) (size 1.7 1.7) (drill 1) (layers "*.Cu" "*.Mask") (remove_unused_layers no))
  (pad "H6" thru_hole circle (at 21.35 18.49) (size 1.7 1.7) (drill 1) (layers "*.Cu" "*.Mask") (remove_unused_layers no))
  (pad "H7" thru_hole circle (at 21.35 21.03) (size 1.7 1.7) (drill 1) (layers "*.Cu" "*.Mask") (remove_unused_layers no))
  (pad "H8" thru_hole circle (at 21.35 23.57) (size 1.7 1.7) (drill 1) (layers "*.Cu" "*.Mask") (remove_unused_layers no))
  (pad "H9" thru_hole circle (at 21.35 26.11) (size 1.7 1.7) (drill 1) (layers "*.Cu" "*.Mask") (remove_unused_layers no))
  (pad "H10" thru_hole circle (at 21.35 28.65) (size 1.7 1.7) (drill 1) (layers "*.Cu" "*.Mask") (remove_unused_layers no))
  (pad "H11" thru_hole circle (at 21.35 31.19) (size 1.7 1.7) (drill 1) (layers "*.Cu" "*.Mask") (remove_unused_layers no))
  (pad "H12" thru_hole circle (at 21.35 33.73) (size 1.7 1.7) (drill 1) (layers "*.Cu" "*.Mask") (remove_unused_layers no))
  (pad "H13" thru_hole circle (at 21.35 36.27) (size 1.7 1.7) (drill 1) (layers "*.Cu" "*.Mask") (remove_unused_layers no))
  (pad "H14" thru_hole circle (at 21.35 38.81) (size 1.7 1.7) (drill 1) (layers "*.Cu" "*.Mask") (remove_unused_layers no))
  (pad "H15" thru_hole circle (at 21.35 41.35) (size 1.7 1.7) (drill 1) (layers "*.Cu" "*.Mask") (remove_unused_layers no))
  (pad "H16" thru_hole circle (at 21.35 43.89) (size 1.7 1.7) (drill 1) (layers "*.Cu" "*.Mask") (remove_unused_layers no))
  (pad "H17" thru_hole circle (at 21.35 46.43) (size 1.7 1.7) (drill 1) (layers "*.Cu" "*.Mask") (remove_unused_layers no))
  (pad "H18" thru_hole circle (at 21.35 48.97) (size 1.7 1.7) (drill 1) (layers "*.Cu" "*.Mask") (remove_unused_layers no))
  (pad "H19" thru_hole circle (at 21.35 51.51) (size 1.7 1.7) (drill 1) (layers "*.Cu" "*.Mask") (remove_unused_layers no))
  (pad "H20" thru_hole circle (at 21.35 54.05) (size 1.7 1.7) (drill 1) (layers "*.Cu" "*.Mask") (remove_unused_layers no))
  (pad "H21" thru_hole circle (at 21.35 56.59) (size 1.7 1.7) (drill 1) (layers "*.Cu" "*.Mask") (remove_unused_layers no))
  (pad "H22" thru_hole circle (at 21.35 59.13) (size 1.7 1.7) (drill 1) (layers "*.Cu" "*.Mask") (remove_unused_layers no))
  (pad "H23" thru_hole circle (at 21.35 61.67) (size 1.7 1.7) (drill 1) (layers "*.Cu" "*.Mask") (remove_unused_layers no) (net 4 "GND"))
  (pad "H24" thru_hole circle (at 21.35 64.21) (size 1.7 1.7) (drill 1) (layers "*.Cu" "*.Mask") (remove_unused_layers no))
  (pad "I1" thru_hole circle (at 23.89 5.79) (size 1.7 1.7) (drill 1) (layers "*.Cu" "*.Mask") (remove_unused_layers no))
  (pad "I2" thru_hole circle (at 23.89 8.33) (size 1.7 1.7) (drill 1) (layers "*.Cu" "*.Mask") (remove_unused_layers no))
  (pad "I3" thru_hole circle (at 23.89 10.87) (size 1.7 1.7) (drill 1) (layers "*.Cu" "*.Mask") (remove_unused_layers no))
  (pad "I4" thru_hole circle (at 23.89 13.41) (size 1.7 1.7) (drill 1) (layers "*.Cu" "*.Mask") (remove_unused_layers no))
  (pad "I5" thru_hole circle (at 23.89 15.95) (size 1.7 1.7) (drill 1) (layers "*.Cu" "*.Mask") (remove_unused_layers no))
  (pad "I6" thru_hole circle (at 23.89 18.49) (size 1.7 1.7) (drill 1) (layers "*.Cu" "*.Mask") (remove_unused_layers no) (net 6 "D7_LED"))
  (pad "I7" thru_hole circle (at 23.89 21.03) (size 1.7 1.7) (drill 1) (layers "*.Cu" "*.Mask") (remove_unused_layers no))
  (pad "I8" thru_hole circle (at 23.89 23.57) (size 1.7 1.7) (drill 1) (layers "*.Cu" "*.Mask") (remove_unused_layers no))
  (pad "I9" thru_hole circle (at 23.89 26.11) (size 1.7 1.7) (drill 1) (layers "*.Cu" "*.Mask") (remove_unused_layers no))
  (pad "I10" thru_hole circle (at 23.89 28.65) (size 1.7 1.7) (drill 1) (layers "*.Cu" "*.Mask") (remove_unused_layers no))
  (pad "I11" thru_hole circle (at 23.89 31.19) (size 1.7 1.7) (drill 1) (layers "*.Cu" "*.Mask") (remove_unused_layers no) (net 5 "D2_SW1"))
  (pad "I12" thru_hole circle (at 23.89 33.73) (size 1.7 1.7) (drill 1) (layers "*.Cu" "*.Mask") (remove_unused_layers no))
  (pad "I13" thru_hole circle (at 23.89 36.27) (size 1.7 1.7) (drill 1) (layers "*.Cu" "*.Mask") (remove_unused_layers no))
  (pad "I14" thru_hole circle (at 23.89 38.81) (size 1.7 1.7) (drill 1) (layers "*.Cu" "*.Mask") (remove_unused_layers no))
  (pad "I15" thru_hole circle (at 23.89 41.35) (size 1.7 1.7) (drill 1) (layers "*.Cu" "*.Mask") (remove_unused_layers no))
  (pad "I16" thru_hole circle (at 23.89 43.89) (size 1.7 1.7) (drill 1) (layers "*.Cu" "*.Mask") (remove_unused_layers no))
  (pad "I17" thru_hole circle (at 23.89 46.43) (size 1.7 1.7) (drill 1) (layers "*.Cu" "*.Mask") (remove_unused_layers no))
  (pad "I18" thru_hole circle (at 23.89 48.97) (size 1.7 1.7) (drill 1) (layers "*.Cu" "*.Mask") (remove_unused_layers no))
  (pad "I19" thru_hole circle (at 23.89 51.51) (size 1.7 1.7) (drill 1) (layers "*.Cu" "*.Mask") (remove_unused_layers no))
  (pad "I20" thru_hole circle (at 23.89 54.05) (size 1.7 1.7) (drill 1) (layers "*.Cu" "*.Mask") (remove_unused_layers no))
  (pad "I21" thru_hole circle (at 23.89 56.59) (size 1.7 1.7) (drill 1) (layers "*.Cu" "*.Mask") (remove_unused_layers no))
  (pad "I22" thru_hole circle (at 23.89 59.13) (size 1.7 1.7) (drill 1) (layers "*.Cu" "*.Mask") (remove_unused_layers no) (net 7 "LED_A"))
  (pad "I23" thru_hole circle (at 23.89 61.67) (size 1.7 1.7) (drill 1) (layers "*.Cu" "*.Mask") (remove_unused_layers no) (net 4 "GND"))
  (pad "I24" thru_hole circle (at 23.89 64.21) (size 1.7 1.7) (drill 1) (layers "*.Cu" "*.Mask") (remove_unused_layers no))
  (pad "J1" thru_hole circle (at 26.43 5.79) (size 1.7 1.7) (drill 1) (layers "*.Cu" "*.Mask") (remove_unused_layers no))
  (pad "J2" thru_hole circle (at 26.43 8.33) (size 1.7 1.7) (drill 1) (layers "*.Cu" "*.Mask") (remove_unused_layers no))
  (pad "J3" thru_hole circle (at 26.43 10.87) (size 1.7 1.7) (drill 1) (layers "*.Cu" "*.Mask") (remove_unused_layers no))
  (pad "J4" thru_hole circle (at 26.43 13.41) (size 1.7 1.7) (drill 1) (layers "*.Cu" "*.Mask") (remove_unused_layers no))
  (pad "J5" thru_hole circle (at 26.43 15.95) (size 1.7 1.7) (drill 1) (layers "*.Cu" "*.Mask") (remove_unused_layers no))
  (pad "J6" thru_hole circle (at 26.43 18.49) (size 1.7 1.7) (drill 1) (layers "*.Cu" "*.Mask") (remove_unused_layers no) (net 6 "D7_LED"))
  (pad "J7" thru_hole circle (at 26.43 21.03) (size 1.7 1.7) (drill 1) (layers "*.Cu" "*.Mask") (remove_unused_layers no))
  (pad "J8" thru_hole circle (at 26.43 23.57) (size 1.7 1.7) (drill 1) (layers "*.Cu" "*.Mask") (remove_unused_layers no))
  (pad "J9" thru_hole circle (at 26.43 26.11) (size 1.7 1.7) (drill 1) (layers "*.Cu" "*.Mask") (remove_unused_layers no))
  (pad "J10" thru_hole circle (at 26.43 28.65) (size 1.7 1.7) (drill 1) (layers "*.Cu" "*.Mask") (remove_unused_layers no))
  (pad "J11" thru_hole circle (at 26.43 31.19) (size 1.7 1.7) (drill 1) (layers "*.Cu" "*.Mask") (remove_unused_layers no) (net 5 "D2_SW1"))
  (pad "J12" thru_hole circle (at 26.43 33.73) (size 1.7 1.7) (drill 1) (layers "*.Cu" "*.Mask") (remove_unused_layers no))
  (pad "J13" thru_hole circle (at 26.43 36.27) (size 1.7 1.7) (drill 1) (layers "*.Cu" "*.Mask") (remove_unused_layers no))
  (pad "J14" thru_hole circle (at 26.43 38.81) (size 1.7 1.7) (drill 1) (layers "*.Cu" "*.Mask") (remove_unused_layers no))
  (pad "J15" thru_hole circle (at 26.43 41.35) (size 1.7 1.7) (drill 1) (layers "*.Cu" "*.Mask") (remove_unused_layers no))
  (pad "J16" thru_hole circle (at 26.43 43.89) (size 1.7 1.7) (drill 1) (layers "*.Cu" "*.Mask") (remove_unused_layers no))
  (pad "J17" thru_hole circle (at 26.43 46.43) (size 1.7 1.7) (drill 1) (layers "*.Cu" "*.Mask") (remove_unused_layers no) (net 6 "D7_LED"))
  (pad "J18" thru_hole circle (at 26.43 48.97) (size 1.7 1.7) (drill 1) (layers "*.Cu" "*.Mask") (remove_unused_layers no) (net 6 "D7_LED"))
  (pad "J19" thru_hole circle (at 26.43 51.51) (size 1.7 1.7) (drill 1) (layers "*.Cu" "*.Mask") (remove_unused_layers no))
  (pad "J20" thru_hole circle (at 26.43 54.05) (size 1.7 1.7) (drill 1) (layers "*.Cu" "*.Mask") (remove_unused_layers no))
  (pad "J21" thru_hole circle (at 26.43 56.59) (size 1.7 1.7) (drill 1) (layers "*.Cu" "*.Mask") (remove_unused_layers no))
  (pad "J22" thru_hole circle (at 26.43 59.13) (size 1.7 1.7) (drill 1) (layers "*.Cu" "*.Mask") (remove_unused_layers no) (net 7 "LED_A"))
  (pad "J23" thru_hole circle (at 26.43 61.67) (size 1.7 1.7) (drill 1) (layers "*.Cu" "*.Mask") (remove_unused_layers no))
  (pad "J24" thru_hole circle (at 26.43 64.21) (size 1.7 1.7) (drill 1) (layers "*.Cu" "*.Mask") (remove_unused_layers no))
  (pad "" np_thru_hole circle (at 2.3 2.3) (size 2 2) (drill 2) (layers "*.Cu" "*.Mask"))
  (pad "" np_thru_hole circle (at 27.7 2.3) (size 2 2) (drill 2) (layers "*.Cu" "*.Mask"))
  (pad "" np_thru_hole circle (at 2.3 67.7) (size 2 2) (drill 2) (layers "*.Cu" "*.Mask"))
  (pad "" np_thru_hole circle (at 27.7 67.7) (size 2 2) (drill 2) (layers "*.Cu" "*.Mask")))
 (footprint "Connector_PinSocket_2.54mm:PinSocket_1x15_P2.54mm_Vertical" (layer "F.Cu") (at 108.65 65.79 0)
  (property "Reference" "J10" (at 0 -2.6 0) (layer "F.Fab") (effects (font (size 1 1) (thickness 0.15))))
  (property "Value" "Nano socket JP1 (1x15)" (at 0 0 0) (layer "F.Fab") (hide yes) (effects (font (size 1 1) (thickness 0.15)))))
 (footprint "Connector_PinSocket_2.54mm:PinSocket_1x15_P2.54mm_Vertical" (layer "F.Cu") (at 123.89 65.79 0)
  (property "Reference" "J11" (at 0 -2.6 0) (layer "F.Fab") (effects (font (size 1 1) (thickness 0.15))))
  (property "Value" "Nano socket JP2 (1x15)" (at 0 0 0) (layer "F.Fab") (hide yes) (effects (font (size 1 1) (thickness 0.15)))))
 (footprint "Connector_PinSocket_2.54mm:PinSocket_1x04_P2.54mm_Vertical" (layer "F.Cu") (at 103.57 111.51 90)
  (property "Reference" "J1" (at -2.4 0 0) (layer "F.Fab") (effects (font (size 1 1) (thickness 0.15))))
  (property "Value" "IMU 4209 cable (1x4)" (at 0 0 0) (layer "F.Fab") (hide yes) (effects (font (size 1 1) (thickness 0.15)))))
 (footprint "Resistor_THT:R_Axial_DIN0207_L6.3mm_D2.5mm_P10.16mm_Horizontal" (layer "F.Cu") (at 126.43 108.97 -90)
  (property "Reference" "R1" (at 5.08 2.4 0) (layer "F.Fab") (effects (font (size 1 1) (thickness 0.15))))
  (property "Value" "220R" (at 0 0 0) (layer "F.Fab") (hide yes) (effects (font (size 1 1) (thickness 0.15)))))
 (gr_rect (start 100 60) (end 130 130) (stroke (width 0.1) (type default)) (fill none) (layer "Edge.Cuts"))
 (segment (start 106.11 68.33) (end 104.84 69.6) (width 0.3) (layer "F.Cu") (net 1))
 (segment (start 104.84 69.6) (end 102 69.6) (width 0.3) (layer "F.Cu") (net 1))
 (segment (start 102 69.6) (end 101.2 70.4) (width 0.3) (layer "F.Cu") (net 1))
 (segment (start 101.2 70.4) (end 101.2 108.17) (width 0.3) (layer "F.Cu") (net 1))
 (segment (start 101.2 108.17) (end 102 108.97) (width 0.3) (layer "F.Cu") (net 1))
 (segment (start 102 108.97) (end 103.57 108.97) (width 0.3) (layer "F.Cu") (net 1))
 (segment (start 106.11 83.57) (end 104.84 84.84) (width 0.3) (layer "F.Cu") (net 2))
 (segment (start 104.84 84.84) (end 104.84 107.7) (width 0.3) (layer "F.Cu") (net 2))
 (segment (start 104.84 107.7) (end 106.11 108.97) (width 0.3) (layer "F.Cu") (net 2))
 (segment (start 106.11 86.11) (end 107.38 87.38) (width 0.3) (layer "F.Cu") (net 3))
 (segment (start 107.38 87.38) (end 107.38 107.7) (width 0.3) (layer "F.Cu") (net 3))
 (segment (start 107.38 107.7) (end 108.65 108.97) (width 0.3) (layer "F.Cu") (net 3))
 (segment (start 126.43 78.49) (end 127.8 78.49) (width 0.3) (layer "F.Cu") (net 6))
 (segment (start 127.8 78.49) (end 128.7 79.39) (width 0.3) (layer "F.Cu") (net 6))
 (segment (start 128.7 79.39) (end 128.7 105.53) (width 0.3) (layer "F.Cu") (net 6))
 (segment (start 128.7 105.53) (end 127.8 106.43) (width 0.3) (layer "F.Cu") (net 6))
 (segment (start 127.8 106.43) (end 126.43 106.43) (width 0.3) (layer "F.Cu") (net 6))
 (segment (start 126.43 91.19) (end 127.5 91.19) (width 0.3) (layer "F.Cu") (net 5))
 (segment (start 127.5 91.19) (end 127.9 91.59) (width 0.3) (layer "F.Cu") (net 5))
 (segment (start 127.9 91.59) (end 127.9 104.76) (width 0.3) (layer "F.Cu") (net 5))
 (segment (start 127.9 104.76) (end 127.5 105.16) (width 0.3) (layer "F.Cu") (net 5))
 (segment (start 127.5 105.16) (end 120.08 105.16) (width 0.3) (layer "F.Cu") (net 5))
 (segment (start 120.08 105.16) (end 120.08 115.32) (width 0.3) (layer "F.Cu") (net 5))
 (segment (start 120.08 115.32) (end 118.81 116.59) (width 0.3) (layer "F.Cu") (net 5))
 (segment (start 106.11 68.33) (end 108.65 68.33) (width 0.8) (layer "B.Cu") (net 1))
 (segment (start 106.11 83.57) (end 108.65 83.57) (width 0.8) (layer "B.Cu") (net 2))
 (segment (start 106.11 86.11) (end 108.65 86.11) (width 0.8) (layer "B.Cu") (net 3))
 (segment (start 108.65 98.81) (end 111.19 98.81) (width 0.8) (layer "B.Cu") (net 4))
 (segment (start 126.43 78.49) (end 123.89 78.49) (width 0.8) (layer "B.Cu") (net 6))
 (segment (start 126.43 91.19) (end 123.89 91.19) (width 0.8) (layer "B.Cu") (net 5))
 (segment (start 126.43 106.43) (end 126.43 108.97) (width 0.8) (layer "B.Cu") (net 6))
 (segment (start 126.43 119.13) (end 123.89 119.13) (width 0.8) (layer "B.Cu") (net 7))
 (segment (start 118.81 116.59) (end 118.81 119.13) (width 0.8) (layer "B.Cu") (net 5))
 (segment (start 103.57 108.97) (end 103.57 119.13) (width 0.8) (layer "B.Cu") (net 1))
 (segment (start 106.11 108.97) (end 106.11 119.13) (width 0.8) (layer "B.Cu") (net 2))
 (segment (start 108.65 108.97) (end 108.65 119.13) (width 0.8) (layer "B.Cu") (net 3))
 (segment (start 111.19 98.81) (end 111.19 121.67) (width 0.8) (layer "B.Cu") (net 4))
 (segment (start 111.19 121.67) (end 123.89 121.67) (width 0.8) (layer "B.Cu") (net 4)))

